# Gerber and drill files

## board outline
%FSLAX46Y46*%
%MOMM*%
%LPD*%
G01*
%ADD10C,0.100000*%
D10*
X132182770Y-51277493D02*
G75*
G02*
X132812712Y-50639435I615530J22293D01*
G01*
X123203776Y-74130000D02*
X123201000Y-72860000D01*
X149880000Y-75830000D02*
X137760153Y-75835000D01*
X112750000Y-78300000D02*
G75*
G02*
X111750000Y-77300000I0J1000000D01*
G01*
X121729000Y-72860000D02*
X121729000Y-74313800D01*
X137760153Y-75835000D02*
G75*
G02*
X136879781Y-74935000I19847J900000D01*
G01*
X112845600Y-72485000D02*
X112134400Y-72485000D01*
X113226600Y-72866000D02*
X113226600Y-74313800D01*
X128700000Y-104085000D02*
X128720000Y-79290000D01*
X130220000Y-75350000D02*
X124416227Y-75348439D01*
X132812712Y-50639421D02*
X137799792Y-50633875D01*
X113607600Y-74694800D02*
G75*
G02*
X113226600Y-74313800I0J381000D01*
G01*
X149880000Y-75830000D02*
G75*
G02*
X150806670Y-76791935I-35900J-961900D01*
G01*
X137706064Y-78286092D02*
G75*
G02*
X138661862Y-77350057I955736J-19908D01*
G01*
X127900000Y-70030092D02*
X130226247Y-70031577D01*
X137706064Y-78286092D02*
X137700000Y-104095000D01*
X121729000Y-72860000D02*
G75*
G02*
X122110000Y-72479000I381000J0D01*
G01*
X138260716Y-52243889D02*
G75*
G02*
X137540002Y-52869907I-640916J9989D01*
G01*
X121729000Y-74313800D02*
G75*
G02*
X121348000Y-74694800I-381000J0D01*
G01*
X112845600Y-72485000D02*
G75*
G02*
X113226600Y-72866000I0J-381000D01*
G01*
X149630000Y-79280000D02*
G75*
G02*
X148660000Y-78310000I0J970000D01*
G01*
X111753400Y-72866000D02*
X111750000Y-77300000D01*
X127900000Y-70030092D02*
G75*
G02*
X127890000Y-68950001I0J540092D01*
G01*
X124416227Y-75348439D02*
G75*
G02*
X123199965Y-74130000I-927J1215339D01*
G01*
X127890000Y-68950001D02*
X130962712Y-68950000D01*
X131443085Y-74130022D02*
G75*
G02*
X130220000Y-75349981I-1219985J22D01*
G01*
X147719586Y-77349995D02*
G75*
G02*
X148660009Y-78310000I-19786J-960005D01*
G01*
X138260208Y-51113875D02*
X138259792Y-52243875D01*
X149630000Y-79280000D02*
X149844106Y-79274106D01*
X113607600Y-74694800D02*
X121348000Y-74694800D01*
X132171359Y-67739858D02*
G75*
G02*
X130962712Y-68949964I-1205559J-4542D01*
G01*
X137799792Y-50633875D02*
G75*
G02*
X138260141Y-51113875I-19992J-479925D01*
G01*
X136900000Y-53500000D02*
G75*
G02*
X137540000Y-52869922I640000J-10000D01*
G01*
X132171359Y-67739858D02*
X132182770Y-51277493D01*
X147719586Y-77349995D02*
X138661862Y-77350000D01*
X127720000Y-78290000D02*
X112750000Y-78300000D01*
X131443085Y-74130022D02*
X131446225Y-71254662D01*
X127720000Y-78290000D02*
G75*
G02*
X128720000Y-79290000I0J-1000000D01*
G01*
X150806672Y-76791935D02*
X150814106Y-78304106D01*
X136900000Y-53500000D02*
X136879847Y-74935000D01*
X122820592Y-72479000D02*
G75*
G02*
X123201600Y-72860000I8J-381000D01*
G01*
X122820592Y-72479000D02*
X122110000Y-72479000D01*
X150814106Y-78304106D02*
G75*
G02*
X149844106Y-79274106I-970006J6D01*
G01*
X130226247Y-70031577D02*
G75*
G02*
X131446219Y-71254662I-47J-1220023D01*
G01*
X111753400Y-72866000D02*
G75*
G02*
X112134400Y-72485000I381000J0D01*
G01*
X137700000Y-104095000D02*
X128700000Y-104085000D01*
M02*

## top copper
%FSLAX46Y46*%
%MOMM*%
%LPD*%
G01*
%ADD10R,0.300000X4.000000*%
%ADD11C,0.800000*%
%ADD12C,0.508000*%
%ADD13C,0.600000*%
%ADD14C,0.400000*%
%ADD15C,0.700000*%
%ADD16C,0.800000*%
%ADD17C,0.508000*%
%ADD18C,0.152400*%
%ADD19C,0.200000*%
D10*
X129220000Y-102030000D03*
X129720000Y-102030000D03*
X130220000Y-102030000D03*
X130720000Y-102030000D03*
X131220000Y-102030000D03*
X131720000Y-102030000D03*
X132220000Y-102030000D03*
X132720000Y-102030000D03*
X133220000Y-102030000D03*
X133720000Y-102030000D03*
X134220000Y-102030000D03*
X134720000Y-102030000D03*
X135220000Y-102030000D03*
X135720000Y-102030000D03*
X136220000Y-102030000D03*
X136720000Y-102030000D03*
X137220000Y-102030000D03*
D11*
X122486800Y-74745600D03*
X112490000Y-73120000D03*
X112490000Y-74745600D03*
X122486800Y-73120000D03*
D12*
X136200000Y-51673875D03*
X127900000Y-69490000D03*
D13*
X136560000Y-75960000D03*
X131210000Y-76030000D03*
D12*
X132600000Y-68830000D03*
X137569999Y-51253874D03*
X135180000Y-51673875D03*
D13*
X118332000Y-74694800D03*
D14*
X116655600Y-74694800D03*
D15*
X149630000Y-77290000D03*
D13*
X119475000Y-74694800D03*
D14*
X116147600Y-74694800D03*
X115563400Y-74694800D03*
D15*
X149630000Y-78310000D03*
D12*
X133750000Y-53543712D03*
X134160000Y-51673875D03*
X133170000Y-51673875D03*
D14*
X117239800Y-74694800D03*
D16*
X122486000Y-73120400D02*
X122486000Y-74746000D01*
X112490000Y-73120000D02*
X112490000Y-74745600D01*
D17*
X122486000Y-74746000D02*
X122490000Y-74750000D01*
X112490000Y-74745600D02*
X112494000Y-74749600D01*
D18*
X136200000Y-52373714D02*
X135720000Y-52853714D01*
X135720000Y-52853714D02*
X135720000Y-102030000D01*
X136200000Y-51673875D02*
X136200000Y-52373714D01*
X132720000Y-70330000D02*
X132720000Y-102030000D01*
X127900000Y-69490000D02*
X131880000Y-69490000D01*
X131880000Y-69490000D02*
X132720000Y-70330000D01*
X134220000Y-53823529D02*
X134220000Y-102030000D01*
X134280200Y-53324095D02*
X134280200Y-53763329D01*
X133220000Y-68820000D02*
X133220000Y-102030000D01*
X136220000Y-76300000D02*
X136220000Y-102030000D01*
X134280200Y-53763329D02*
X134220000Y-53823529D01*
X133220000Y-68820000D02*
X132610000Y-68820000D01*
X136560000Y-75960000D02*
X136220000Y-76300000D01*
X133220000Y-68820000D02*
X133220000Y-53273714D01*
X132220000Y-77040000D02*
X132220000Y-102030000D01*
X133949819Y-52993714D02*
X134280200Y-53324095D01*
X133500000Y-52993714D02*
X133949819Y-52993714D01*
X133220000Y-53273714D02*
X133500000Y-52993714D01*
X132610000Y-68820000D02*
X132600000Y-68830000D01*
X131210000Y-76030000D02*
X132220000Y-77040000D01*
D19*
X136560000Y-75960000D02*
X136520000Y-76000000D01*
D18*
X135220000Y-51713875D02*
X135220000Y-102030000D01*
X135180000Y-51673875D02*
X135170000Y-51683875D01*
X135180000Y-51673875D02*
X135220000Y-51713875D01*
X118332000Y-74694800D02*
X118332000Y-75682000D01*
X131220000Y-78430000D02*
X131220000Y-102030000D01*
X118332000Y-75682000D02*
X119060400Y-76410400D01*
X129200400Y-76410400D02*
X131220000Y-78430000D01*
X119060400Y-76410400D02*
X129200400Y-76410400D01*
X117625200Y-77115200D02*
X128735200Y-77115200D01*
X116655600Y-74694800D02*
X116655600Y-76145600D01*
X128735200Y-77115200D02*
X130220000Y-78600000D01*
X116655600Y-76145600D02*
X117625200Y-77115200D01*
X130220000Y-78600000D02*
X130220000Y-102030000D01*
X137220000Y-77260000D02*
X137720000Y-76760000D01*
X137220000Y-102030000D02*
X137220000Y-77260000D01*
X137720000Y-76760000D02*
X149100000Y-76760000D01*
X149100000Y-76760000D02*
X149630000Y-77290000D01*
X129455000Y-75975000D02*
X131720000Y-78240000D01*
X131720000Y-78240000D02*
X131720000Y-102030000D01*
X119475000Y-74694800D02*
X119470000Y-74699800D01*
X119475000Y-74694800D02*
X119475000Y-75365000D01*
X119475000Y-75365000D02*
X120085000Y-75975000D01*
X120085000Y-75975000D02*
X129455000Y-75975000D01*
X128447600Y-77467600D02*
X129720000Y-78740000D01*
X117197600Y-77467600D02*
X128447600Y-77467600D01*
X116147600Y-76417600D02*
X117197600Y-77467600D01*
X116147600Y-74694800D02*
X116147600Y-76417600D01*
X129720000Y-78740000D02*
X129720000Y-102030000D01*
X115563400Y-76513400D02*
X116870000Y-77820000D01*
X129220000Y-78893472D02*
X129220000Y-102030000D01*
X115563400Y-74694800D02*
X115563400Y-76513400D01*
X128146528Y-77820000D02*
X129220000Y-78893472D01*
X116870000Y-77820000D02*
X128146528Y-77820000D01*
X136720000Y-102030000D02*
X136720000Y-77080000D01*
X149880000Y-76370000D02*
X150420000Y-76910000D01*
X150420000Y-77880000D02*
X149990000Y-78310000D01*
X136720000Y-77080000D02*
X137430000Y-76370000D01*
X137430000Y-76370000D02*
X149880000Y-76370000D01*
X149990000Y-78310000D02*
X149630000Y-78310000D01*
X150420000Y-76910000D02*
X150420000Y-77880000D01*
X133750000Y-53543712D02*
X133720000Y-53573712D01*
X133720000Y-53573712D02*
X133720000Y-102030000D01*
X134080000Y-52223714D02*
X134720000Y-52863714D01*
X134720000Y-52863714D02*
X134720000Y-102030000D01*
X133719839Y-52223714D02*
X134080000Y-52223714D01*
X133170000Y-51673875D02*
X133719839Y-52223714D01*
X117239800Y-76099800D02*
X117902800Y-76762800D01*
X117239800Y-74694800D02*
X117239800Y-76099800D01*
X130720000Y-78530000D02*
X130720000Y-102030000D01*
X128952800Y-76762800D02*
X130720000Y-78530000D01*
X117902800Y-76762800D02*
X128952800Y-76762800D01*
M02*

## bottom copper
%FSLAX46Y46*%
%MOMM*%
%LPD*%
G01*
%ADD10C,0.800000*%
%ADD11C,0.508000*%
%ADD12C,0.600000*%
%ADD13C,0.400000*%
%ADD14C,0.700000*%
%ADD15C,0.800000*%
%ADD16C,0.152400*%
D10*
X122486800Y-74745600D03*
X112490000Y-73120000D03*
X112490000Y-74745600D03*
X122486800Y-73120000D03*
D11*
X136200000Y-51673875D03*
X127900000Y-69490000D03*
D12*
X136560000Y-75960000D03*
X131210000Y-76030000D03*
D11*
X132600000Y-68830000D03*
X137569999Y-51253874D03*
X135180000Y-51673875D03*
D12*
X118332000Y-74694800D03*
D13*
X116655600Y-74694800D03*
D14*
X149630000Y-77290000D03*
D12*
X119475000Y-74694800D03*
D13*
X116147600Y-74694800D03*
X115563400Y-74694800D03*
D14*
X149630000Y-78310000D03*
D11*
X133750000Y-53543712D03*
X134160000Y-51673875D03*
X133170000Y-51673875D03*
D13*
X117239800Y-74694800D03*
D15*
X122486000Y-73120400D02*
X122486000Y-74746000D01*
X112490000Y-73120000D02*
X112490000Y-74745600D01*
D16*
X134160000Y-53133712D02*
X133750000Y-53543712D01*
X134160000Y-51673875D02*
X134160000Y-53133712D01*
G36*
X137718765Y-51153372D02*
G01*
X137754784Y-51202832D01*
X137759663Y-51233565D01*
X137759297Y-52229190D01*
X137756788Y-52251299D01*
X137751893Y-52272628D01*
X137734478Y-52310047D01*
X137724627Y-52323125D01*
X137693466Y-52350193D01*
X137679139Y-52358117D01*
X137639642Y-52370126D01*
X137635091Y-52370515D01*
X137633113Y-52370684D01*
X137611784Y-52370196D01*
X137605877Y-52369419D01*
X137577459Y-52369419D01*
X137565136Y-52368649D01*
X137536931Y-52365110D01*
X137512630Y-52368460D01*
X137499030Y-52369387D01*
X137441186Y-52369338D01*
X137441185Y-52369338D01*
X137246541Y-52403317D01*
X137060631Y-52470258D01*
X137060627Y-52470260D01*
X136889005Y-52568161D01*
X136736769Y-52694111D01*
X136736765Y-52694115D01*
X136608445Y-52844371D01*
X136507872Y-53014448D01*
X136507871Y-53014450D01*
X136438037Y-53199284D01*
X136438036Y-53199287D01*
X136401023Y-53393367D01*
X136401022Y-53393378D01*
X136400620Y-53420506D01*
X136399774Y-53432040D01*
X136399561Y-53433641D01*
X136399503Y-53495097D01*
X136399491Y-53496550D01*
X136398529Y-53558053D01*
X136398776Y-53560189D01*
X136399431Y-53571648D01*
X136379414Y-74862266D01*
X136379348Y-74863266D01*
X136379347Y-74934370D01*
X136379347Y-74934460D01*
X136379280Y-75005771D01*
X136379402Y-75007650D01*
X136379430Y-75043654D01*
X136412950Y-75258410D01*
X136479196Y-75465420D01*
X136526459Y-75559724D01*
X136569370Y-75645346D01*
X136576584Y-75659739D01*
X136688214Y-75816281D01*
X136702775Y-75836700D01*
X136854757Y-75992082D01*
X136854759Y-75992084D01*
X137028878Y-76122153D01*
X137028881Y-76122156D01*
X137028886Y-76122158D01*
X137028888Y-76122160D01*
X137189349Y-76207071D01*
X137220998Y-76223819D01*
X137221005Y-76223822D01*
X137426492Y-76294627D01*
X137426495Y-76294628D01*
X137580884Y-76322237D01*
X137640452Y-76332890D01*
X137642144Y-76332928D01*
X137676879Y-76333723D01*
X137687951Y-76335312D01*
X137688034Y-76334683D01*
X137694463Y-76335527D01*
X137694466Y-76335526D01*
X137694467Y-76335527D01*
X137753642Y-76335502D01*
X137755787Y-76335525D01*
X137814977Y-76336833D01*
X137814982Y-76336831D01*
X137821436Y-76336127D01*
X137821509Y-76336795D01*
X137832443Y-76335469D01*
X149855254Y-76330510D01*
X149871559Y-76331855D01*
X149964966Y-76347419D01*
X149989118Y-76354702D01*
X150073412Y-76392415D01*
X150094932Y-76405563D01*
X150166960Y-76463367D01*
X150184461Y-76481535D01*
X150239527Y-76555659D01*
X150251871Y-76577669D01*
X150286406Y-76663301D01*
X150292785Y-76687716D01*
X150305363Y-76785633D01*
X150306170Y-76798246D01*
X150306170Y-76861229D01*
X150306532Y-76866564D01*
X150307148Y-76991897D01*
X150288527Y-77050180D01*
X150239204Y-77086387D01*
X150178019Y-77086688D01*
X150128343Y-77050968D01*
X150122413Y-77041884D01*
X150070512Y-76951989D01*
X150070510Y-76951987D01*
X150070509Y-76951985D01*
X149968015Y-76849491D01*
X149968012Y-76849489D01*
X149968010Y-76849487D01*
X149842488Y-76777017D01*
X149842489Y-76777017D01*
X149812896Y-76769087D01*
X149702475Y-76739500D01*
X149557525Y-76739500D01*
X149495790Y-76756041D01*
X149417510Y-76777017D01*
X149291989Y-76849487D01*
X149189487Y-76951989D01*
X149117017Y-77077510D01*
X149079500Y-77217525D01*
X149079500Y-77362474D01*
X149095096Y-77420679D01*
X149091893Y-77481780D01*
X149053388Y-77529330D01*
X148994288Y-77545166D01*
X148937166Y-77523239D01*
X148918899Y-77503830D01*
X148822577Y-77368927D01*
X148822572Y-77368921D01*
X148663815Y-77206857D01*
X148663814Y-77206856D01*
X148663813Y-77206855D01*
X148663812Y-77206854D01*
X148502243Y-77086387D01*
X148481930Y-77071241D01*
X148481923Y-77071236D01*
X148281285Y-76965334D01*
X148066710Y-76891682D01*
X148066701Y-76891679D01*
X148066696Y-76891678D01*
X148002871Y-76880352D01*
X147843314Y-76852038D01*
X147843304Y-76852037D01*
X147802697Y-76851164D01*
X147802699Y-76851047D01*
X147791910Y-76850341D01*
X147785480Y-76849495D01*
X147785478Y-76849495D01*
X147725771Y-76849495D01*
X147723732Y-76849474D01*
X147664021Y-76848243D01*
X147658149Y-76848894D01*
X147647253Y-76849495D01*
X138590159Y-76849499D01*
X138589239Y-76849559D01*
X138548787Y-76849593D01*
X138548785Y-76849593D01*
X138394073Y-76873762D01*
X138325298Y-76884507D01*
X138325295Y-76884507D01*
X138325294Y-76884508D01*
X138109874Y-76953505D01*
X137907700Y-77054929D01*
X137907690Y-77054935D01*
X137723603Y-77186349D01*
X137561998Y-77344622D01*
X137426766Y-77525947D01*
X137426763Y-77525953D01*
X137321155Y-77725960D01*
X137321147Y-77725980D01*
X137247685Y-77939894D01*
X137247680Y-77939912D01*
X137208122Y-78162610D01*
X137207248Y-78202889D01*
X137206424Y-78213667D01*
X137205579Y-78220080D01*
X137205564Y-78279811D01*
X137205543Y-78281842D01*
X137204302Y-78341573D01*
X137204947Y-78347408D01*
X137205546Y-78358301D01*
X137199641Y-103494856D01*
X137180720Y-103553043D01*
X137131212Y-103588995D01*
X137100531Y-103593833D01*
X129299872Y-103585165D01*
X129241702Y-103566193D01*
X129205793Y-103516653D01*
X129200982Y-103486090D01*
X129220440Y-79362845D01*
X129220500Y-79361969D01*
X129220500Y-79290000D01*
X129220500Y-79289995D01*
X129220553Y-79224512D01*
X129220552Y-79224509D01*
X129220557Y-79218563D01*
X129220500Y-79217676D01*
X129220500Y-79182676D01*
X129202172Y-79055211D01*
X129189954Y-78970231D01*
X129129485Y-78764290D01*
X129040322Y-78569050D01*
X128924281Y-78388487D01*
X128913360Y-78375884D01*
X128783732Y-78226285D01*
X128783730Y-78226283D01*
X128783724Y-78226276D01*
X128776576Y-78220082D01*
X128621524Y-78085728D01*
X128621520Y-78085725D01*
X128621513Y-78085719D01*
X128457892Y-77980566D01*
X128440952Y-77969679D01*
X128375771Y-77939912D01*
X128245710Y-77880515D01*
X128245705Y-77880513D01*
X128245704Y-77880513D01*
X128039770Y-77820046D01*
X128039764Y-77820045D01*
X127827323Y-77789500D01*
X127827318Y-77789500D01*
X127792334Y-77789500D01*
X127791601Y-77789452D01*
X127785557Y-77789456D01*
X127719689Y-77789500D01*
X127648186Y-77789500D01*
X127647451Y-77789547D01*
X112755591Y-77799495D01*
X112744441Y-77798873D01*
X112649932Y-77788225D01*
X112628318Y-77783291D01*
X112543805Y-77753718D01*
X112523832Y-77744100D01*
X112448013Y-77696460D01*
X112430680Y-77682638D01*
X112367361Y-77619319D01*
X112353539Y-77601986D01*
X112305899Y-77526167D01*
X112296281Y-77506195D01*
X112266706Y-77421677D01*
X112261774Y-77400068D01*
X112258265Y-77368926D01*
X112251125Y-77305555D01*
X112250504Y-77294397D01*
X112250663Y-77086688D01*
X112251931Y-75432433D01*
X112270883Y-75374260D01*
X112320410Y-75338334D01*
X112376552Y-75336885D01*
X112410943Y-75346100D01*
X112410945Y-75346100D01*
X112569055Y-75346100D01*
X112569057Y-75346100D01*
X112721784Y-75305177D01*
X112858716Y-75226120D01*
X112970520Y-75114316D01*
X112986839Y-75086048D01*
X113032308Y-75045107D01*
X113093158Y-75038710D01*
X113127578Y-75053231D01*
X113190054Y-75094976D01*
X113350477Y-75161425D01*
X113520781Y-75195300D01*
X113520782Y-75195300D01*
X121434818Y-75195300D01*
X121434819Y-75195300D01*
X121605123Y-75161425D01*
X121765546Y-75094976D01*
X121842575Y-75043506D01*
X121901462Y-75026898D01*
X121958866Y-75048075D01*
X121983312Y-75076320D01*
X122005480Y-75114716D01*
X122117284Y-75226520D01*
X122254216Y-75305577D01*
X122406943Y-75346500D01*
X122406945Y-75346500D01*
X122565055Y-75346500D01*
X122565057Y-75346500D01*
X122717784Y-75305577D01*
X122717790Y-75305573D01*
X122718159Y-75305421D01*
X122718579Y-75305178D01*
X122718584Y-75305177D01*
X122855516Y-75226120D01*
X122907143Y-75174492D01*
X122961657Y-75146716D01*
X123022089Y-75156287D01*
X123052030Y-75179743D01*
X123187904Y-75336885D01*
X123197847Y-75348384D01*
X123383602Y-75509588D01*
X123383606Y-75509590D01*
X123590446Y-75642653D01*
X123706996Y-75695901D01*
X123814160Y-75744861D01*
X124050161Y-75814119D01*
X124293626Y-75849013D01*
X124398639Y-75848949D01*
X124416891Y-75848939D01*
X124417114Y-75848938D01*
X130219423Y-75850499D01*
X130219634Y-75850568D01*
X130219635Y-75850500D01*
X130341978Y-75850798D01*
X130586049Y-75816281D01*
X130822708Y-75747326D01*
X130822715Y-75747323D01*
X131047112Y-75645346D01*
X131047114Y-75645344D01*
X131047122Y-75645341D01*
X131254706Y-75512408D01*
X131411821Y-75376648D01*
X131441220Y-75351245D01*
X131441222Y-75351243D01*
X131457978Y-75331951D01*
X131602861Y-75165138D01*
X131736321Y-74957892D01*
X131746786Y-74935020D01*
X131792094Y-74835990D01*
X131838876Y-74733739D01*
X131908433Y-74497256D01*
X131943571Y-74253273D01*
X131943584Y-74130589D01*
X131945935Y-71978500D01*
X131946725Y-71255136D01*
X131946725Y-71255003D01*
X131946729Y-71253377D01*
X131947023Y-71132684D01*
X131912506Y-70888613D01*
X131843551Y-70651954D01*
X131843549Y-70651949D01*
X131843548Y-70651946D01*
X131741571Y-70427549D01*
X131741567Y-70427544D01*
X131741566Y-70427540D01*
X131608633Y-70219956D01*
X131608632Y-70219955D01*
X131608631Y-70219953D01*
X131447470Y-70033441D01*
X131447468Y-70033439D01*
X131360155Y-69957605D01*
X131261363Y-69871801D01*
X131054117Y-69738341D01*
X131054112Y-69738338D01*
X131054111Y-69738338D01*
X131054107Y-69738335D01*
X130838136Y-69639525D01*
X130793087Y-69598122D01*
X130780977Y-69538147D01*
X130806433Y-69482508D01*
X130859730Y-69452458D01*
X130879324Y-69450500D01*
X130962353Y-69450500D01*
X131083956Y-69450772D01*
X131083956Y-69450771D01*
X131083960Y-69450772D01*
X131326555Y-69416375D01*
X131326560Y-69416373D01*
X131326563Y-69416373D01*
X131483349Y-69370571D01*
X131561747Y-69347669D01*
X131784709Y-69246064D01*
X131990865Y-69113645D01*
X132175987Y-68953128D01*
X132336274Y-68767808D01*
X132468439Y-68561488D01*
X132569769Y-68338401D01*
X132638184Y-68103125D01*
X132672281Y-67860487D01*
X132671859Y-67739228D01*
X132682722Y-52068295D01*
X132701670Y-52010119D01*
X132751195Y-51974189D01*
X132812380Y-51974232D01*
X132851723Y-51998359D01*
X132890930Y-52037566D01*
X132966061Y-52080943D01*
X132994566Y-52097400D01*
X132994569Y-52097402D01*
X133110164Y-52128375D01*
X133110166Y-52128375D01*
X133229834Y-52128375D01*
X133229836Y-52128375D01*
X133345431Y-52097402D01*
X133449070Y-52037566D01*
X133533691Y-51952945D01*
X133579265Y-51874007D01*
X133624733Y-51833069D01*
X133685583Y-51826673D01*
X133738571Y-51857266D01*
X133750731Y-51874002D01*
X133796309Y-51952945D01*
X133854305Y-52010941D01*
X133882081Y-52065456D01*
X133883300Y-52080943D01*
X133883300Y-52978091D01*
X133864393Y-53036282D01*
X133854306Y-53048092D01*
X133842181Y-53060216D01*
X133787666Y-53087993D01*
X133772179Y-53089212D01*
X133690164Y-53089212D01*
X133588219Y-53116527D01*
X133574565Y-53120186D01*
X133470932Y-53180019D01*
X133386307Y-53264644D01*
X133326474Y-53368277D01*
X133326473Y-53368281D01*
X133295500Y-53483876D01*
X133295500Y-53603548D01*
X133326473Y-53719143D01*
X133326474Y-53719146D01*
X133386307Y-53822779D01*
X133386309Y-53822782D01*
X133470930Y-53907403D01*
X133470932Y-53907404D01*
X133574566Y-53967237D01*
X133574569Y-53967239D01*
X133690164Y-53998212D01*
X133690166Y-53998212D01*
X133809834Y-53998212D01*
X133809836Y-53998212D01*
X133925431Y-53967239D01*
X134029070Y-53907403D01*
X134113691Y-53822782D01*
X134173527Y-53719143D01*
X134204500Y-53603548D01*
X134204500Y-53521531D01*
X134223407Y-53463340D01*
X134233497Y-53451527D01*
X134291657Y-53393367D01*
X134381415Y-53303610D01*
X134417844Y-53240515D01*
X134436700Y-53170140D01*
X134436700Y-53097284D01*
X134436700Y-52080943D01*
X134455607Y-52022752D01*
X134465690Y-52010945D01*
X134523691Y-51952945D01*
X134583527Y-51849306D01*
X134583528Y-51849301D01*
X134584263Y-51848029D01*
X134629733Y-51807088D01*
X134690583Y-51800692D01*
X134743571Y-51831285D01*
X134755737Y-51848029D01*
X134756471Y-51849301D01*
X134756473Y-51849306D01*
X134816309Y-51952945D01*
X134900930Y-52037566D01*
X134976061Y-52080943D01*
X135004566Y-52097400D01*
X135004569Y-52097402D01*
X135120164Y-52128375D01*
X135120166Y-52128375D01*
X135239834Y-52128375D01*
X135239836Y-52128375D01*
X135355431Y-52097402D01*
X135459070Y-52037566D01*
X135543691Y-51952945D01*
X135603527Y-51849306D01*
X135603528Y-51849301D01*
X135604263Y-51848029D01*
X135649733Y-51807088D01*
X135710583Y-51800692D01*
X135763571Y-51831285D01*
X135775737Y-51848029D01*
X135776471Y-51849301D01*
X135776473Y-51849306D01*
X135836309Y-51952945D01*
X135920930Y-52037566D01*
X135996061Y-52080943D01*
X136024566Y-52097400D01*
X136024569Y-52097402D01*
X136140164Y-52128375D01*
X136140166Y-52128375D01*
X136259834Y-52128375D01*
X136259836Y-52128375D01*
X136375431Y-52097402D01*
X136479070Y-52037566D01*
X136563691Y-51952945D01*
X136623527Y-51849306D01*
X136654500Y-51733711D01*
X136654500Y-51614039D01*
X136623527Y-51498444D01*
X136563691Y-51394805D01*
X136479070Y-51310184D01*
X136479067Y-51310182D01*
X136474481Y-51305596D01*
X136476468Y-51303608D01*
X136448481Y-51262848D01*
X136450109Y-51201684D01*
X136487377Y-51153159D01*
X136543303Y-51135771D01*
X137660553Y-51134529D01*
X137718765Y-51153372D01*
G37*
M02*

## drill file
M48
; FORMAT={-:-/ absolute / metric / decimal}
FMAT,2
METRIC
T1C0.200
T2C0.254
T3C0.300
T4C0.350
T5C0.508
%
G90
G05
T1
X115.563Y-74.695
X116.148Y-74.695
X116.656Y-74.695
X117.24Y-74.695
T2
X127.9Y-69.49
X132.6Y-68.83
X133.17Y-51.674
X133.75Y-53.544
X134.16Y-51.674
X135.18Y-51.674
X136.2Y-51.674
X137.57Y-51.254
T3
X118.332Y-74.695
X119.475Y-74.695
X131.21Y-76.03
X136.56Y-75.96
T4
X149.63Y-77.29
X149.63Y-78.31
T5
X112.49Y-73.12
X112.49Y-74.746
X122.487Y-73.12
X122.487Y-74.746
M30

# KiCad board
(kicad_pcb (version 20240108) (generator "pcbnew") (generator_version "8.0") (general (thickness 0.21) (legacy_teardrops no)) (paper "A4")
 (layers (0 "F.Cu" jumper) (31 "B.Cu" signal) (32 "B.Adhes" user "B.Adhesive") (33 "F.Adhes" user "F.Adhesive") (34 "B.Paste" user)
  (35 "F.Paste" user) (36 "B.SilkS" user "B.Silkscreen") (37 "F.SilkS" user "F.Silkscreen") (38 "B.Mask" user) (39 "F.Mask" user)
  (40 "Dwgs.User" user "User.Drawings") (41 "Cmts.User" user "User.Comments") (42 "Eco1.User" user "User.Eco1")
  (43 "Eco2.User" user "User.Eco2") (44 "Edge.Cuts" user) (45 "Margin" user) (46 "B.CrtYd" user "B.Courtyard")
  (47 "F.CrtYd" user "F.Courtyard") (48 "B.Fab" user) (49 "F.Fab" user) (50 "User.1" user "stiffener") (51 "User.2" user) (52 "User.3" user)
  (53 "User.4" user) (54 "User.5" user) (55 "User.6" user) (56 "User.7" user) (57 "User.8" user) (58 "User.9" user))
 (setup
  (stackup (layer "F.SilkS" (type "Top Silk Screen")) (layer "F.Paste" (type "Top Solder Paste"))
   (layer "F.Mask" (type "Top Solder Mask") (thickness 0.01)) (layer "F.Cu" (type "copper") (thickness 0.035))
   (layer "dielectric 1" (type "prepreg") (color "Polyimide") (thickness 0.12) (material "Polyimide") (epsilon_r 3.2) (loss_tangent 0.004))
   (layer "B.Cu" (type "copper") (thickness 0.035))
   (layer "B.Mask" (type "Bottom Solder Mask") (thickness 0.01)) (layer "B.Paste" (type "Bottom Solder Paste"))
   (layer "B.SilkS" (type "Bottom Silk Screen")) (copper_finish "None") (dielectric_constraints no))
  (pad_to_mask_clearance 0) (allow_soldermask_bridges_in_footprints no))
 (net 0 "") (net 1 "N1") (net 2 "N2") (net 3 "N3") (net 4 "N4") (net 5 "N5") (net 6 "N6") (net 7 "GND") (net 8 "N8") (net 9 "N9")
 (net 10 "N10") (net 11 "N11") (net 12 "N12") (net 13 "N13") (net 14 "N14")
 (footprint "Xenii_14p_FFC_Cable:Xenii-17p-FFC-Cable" (layer "F.Cu") (at 129.22 102.03 90)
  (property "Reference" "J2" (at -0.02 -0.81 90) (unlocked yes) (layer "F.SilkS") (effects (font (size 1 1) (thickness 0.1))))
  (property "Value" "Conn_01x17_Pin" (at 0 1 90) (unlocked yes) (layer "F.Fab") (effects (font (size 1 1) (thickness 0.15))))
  (pad "1" smd rect (at 0 0 90) (size 4 0.3) (layers "F.Cu" "F.Paste" "F.Mask") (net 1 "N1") (thermal_bridge_angle 45))
  (pad "2" smd rect (at 0 0.5 90) (size 4 0.3) (layers "F.Cu" "F.Paste" "F.Mask") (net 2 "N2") (thermal_bridge_angle 45))
  (pad "3" smd rect (at 0 1 90) (size 4 0.3) (layers "F.Cu" "F.Paste" "F.Mask") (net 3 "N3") (thermal_bridge_angle 45))
  (pad "4" smd rect (at 0 1.5 90) (size 4 0.3) (layers "F.Cu" "F.Paste" "F.Mask") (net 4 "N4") (thermal_bridge_angle 45))
  (pad "5" smd rect (at 0 2 90) (size 4 0.3) (layers "F.Cu" "F.Paste" "F.Mask") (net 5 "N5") (thermal_bridge_angle 45))
  (pad "6" smd rect (at 0 2.5 90) (size 4 0.3) (layers "F.Cu" "F.Paste" "F.Mask") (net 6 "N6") (thermal_bridge_angle 45))
  (pad "7" smd rect (at 0 3 90) (size 4 0.3) (layers "F.Cu" "F.Paste" "F.Mask") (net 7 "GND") (thermal_bridge_angle 45))
  (pad "8" smd rect (at 0 3.5 90) (size 4 0.3) (layers "F.Cu" "F.Paste" "F.Mask") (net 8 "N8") (thermal_bridge_angle 45))
  (pad "9" smd rect (at 0 4 90) (size 4 0.3) (layers "F.Cu" "F.Paste" "F.Mask") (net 7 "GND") (thermal_bridge_angle 45))
  (pad "10" smd rect (at 0 4.5 90) (size 4 0.3) (layers "F.Cu" "F.Paste" "F.Mask") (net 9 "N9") (thermal_bridge_angle 45))
  (pad "11" smd rect (at 0 5 90) (size 4 0.3) (layers "F.Cu" "F.Paste" "F.Mask") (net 7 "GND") (thermal_bridge_angle 45))
  (pad "12" smd rect (at 0 5.5 90) (size 4 0.3) (layers "F.Cu" "F.Paste" "F.Mask") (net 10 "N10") (thermal_bridge_angle 45))
  (pad "13" smd rect (at 0 6 90) (size 4 0.3) (layers "F.Cu" "F.Paste" "F.Mask") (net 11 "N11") (thermal_bridge_angle 45))
  (pad "14" smd rect (at 0 6.5 90) (size 4 0.3) (layers "F.Cu" "F.Paste" "F.Mask") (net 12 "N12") (thermal_bridge_angle 45))
  (pad "15" smd rect (at 0 7 90) (size 4 0.3) (layers "F.Cu" "F.Paste" "F.Mask") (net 7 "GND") (thermal_bridge_angle 45))
  (pad "16" smd rect (at 0 7.5 90) (size 4 0.3) (layers "F.Cu" "F.Paste" "F.Mask") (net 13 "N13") (thermal_bridge_angle 45))
  (pad "17" smd rect (at 0 8 90) (size 4 0.3) (layers "F.Cu" "F.Paste" "F.Mask") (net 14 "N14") (thermal_bridge_angle 45)))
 (gr_arc (start 132.18277 51.277493) (mid 132.359996 50.822475) (end 132.812712 50.639421) (stroke (width 0.1) (type default))
  (layer "Edge.Cuts"))
 (gr_line (start 123.203776 74.13) (end 123.201 72.86) (stroke (width 0.1) (type default)) (layer "Edge.Cuts"))
 (gr_line (start 149.88 75.83) (end 137.760153 75.835) (stroke (width 0.1) (type default)) (layer "Edge.Cuts"))
 (gr_arc (start 112.75 78.3) (mid 112.042893 78.007107) (end 111.75 77.3) (stroke (width 0.1) (type default)) (layer "Edge.Cuts"))
 (gr_line (start 121.729 72.86) (end 121.729 74.3138) (stroke (width 0.1) (type default)) (layer "Edge.Cuts"))
 (gr_arc (start 137.760153 75.835) (mid 137.1365 75.564479) (end 136.879847 74.935) (stroke (width 0.1) (type default)) (layer "Edge.Cuts"))
 (gr_line (start 112.8456 72.485) (end 112.1344 72.485) (stroke (width 0.1) (type default)) (layer "Edge.Cuts"))
 (gr_line (start 113.2266 72.866) (end 113.2266 74.3138) (stroke (width 0.1) (type default)) (layer "Edge.Cuts"))
 (gr_line (start 128.7 104.085) (end 128.72 79.29) (stroke (width 0.1) (type default)) (layer "Edge.Cuts"))
 (gr_line (start 130.22 75.35) (end 124.416227 75.348439) (stroke (width 0.1) (type default)) (layer "Edge.Cuts"))
 (gr_line (start 132.812712 50.639421) (end 137.799792 50.633875) (stroke (width 0.1) (type default)) (layer "Edge.Cuts"))
 (gr_arc (start 113.6076 74.6948) (mid 113.338192 74.583208) (end 113.2266 74.3138) (stroke (width 0.1) (type default)) (layer "Edge.Cuts"))
 (gr_arc (start 149.88 75.83) (mid 150.537328 76.124086) (end 150.806672 76.791935) (stroke (width 0.1) (type default)) (layer "Edge.Cuts"))
 (gr_arc (start 137.706064 78.286092) (mid 137.992937 77.622986) (end 138.661862 77.35) (stroke (width 0.1) (type default))
  (layer "Edge.Cuts"))
 (gr_line (start 127.9 70.030092) (end 130.226247 70.031577) (stroke (width 0.1) (type default)) (layer "Edge.Cuts"))
 (gr_line (start 137.706064 78.286092) (end 137.7 104.095) (stroke (width 0.1) (type default)) (layer "Edge.Cuts"))
 (gr_arc (start 121.729 72.86) (mid 121.840592 72.590592) (end 122.11 72.479) (stroke (width 0.1) (type default)) (layer "Edge.Cuts"))
 (gr_arc (start 138.260716 52.243889) (mid 138.040147 52.717837) (end 137.54 52.869921) (stroke (width 0.1) (type default))
  (layer "Edge.Cuts"))
 (gr_arc (start 121.729 74.3138) (mid 121.617408 74.583208) (end 121.348 74.6948) (stroke (width 0.1) (type default)) (layer "Edge.Cuts"))
 (gr_arc (start 112.8456 72.485) (mid 113.115008 72.596592) (end 113.2266 72.866) (stroke (width 0.1) (type default)) (layer "Edge.Cuts"))
 (gr_arc (start 149.63 79.28) (mid 148.944106 78.995894) (end 148.66 78.31) (stroke (width 0.1) (type default)) (layer "Edge.Cuts"))
 (gr_line (start 111.7534 72.866) (end 111.75 77.3) (stroke (width 0.1) (type default)) (layer "Edge.Cuts"))
 (gr_arc (start 127.9 70.030092) (mid 127.359931 69.495) (end 127.89 68.950001) (stroke (width 0.1) (type default)) (layer "Edge.Cuts"))
 (gr_arc (start 124.416227 75.348439) (mid 123.555173 74.991698) (end 123.2 74.13) (stroke (width 0.1) (type default)) (layer "Edge.Cuts"))
 (gr_line (start 127.89 68.950001) (end 130.962712 68.95) (stroke (width 0.1) (type default)) (layer "Edge.Cuts"))
 (gr_arc (start 131.443085 74.130022) (mid 131.084662 74.993775) (end 130.22 75.35) (stroke (width 0.1) (type default)) (layer "Edge.Cuts"))
 (gr_arc (start 147.719586 77.349995) (mid 148.38573 77.638062) (end 148.66 78.31) (stroke (width 0.1) (type default)) (layer "Edge.Cuts"))
 (gr_line (start 138.260208 51.113875) (end 138.259792 52.243875) (stroke (width 0.1) (type default)) (layer "Edge.Cuts"))
 (gr_line (start 149.63 79.28) (end 149.844106 79.274106) (stroke (width 0.1) (type default)) (layer "Edge.Cuts"))
 (gr_line (start 113.6076 74.6948) (end 121.348 74.6948) (stroke (width 0.1) (type default)) (layer "Edge.Cuts"))
 (gr_arc (start 132.171359 67.739858) (mid 131.818778 68.59636) (end 130.962712 68.95) (stroke (width 0.1) (type default))
  (layer "Edge.Cuts"))
 (gr_arc (start 137.799792 50.633875) (mid 138.126516 50.78131) (end 138.260208 51.113875) (stroke (width 0.1) (type default))
  (layer "Edge.Cuts"))
 (gr_arc (start 136.9 53.5) (mid 137.090951 53.053884) (end 137.54 52.869922) (stroke (width 0.1) (type default)) (layer "Edge.Cuts"))
 (gr_line (start 132.171359 67.739858) (end 132.18277 51.277493) (stroke (width 0.1) (type default)) (layer "Edge.Cuts"))
 (gr_line (start 147.719586 77.349995) (end 138.661862 77.35) (stroke (width 0.1) (type default)) (layer "Edge.Cuts"))
 (gr_line (start 127.72 78.29) (end 112.75 78.3) (stroke (width 0.1) (type default)) (layer "Edge.Cuts"))
 (gr_line (start 131.443085 74.130022) (end 131.446225 71.254662) (stroke (width 0.1) (type default)) (layer "Edge.Cuts"))
 (gr_arc (start 127.72 78.29) (mid 128.427107 78.582893) (end 128.72 79.29) (stroke (width 0.1) (type default)) (layer "Edge.Cuts"))
 (gr_line (start 150.806672 76.791935) (end 150.814106 78.304106) (stroke (width 0.1) (type default)) (layer "Edge.Cuts"))
 (gr_line (start 136.9 53.5) (end 136.879847 74.935) (stroke (width 0.1) (type default)) (layer "Edge.Cuts"))
 (gr_arc (start 122.820592 72.479) (mid 123.09 72.590592) (end 123.201592 72.86) (stroke (width 0.1) (type default)) (layer "Edge.Cuts"))
 (gr_line (start 122.820592 72.479) (end 122.11 72.479) (stroke (width 0.1) (type default)) (layer "Edge.Cuts"))
 (gr_arc (start 150.814106 78.304106) (mid 150.529998 78.989998) (end 149.844106 79.274106) (stroke (width 0.1) (type default))
  (layer "Edge.Cuts"))
 (gr_arc (start 130.226247 70.031577) (mid 131.09 70.39) (end 131.446225 71.254662) (stroke (width 0.1) (type default)) (layer "Edge.Cuts"))
 (gr_arc (start 111.7534 72.866) (mid 111.864992 72.596592) (end 112.1344 72.485) (stroke (width 0.1) (type default)) (layer "Edge.Cuts"))
 (gr_line (start 137.7 104.095) (end 128.7 104.085) (stroke (width 0.1) (type default)) (layer "Edge.Cuts"))
 (segment (start 122.486 73.1204) (end 122.486 74.746) (width 0.8) (layer "F.Cu") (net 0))
 (segment (start 112.49 73.12) (end 112.49 74.7456) (width 0.8) (layer "F.Cu") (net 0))
 (segment (start 122.486 74.746) (end 122.49 74.75) (width 0.508) (layer "F.Cu") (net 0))
 (segment (start 112.49 74.7456) (end 112.494 74.7496) (width 0.508) (layer "F.Cu") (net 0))
 (via (at 122.4868 74.7456) (size 0.8) (drill 0.508) (layers "F.Cu" "B.Cu") (free yes) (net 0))
 (via (at 112.49 73.12) (size 0.8) (drill 0.508) (layers "F.Cu" "B.Cu") (free yes) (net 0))
 (via (at 112.49 74.7456) (size 0.8) (drill 0.508) (layers "F.Cu" "B.Cu") (free yes) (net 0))
 (via (at 122.4868 73.12) (size 0.8) (drill 0.508) (layers "F.Cu" "B.Cu") (free yes) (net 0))
 (segment (start 122.486 73.1204) (end 122.486 74.746) (width 0.8) (layer "B.Cu") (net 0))
 (segment (start 112.49 73.12) (end 112.49 74.7456) (width 0.8) (layer "B.Cu") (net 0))
 (segment (start 136.2 52.373714) (end 135.72 52.853714) (width 0.1524) (layer "F.Cu") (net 12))
 (segment (start 135.72 52.853714) (end 135.72 102.03) (width 0.1524) (layer "F.Cu") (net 12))
 (segment (start 136.2 51.673875) (end 136.2 52.373714) (width 0.1524) (layer "F.Cu") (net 12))
 (via (at 136.2 51.673875) (size 0.508) (drill 0.254253) (layers "F.Cu" "B.Cu") (free yes) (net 12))
 (segment (start 132.72 70.33) (end 132.72 102.03) (width 0.1524) (layer "F.Cu") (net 8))
 (segment (start 127.9 69.49) (end 131.88 69.49) (width 0.1524) (layer "F.Cu") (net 8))
 (segment (start 131.88 69.49) (end 132.72 70.33) (width 0.1524) (layer "F.Cu") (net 8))
 (via (at 127.9 69.49) (size 0.508) (drill 0.254253) (layers "F.Cu" "B.Cu") (free yes) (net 8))
 (segment (start 134.22 53.823529) (end 134.22 102.03) (width 0.1524) (layer "F.Cu") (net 7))
 (segment (start 134.2802 53.324095) (end 134.2802 53.763329) (width 0.1524) (layer "F.Cu") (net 7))
 (segment (start 133.22 68.82) (end 133.22 102.03) (width 0.1524) (layer "F.Cu") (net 7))
 (segment (start 136.22 76.3) (end 136.22 102.03) (width 0.1524) (layer "F.Cu") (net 7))
 (segment (start 134.2802 53.763329) (end 134.22 53.823529) (width 0.1524) (layer "F.Cu") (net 7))
 (segment (start 133.22 68.82) (end 132.61 68.82) (width 0.1524) (layer "F.Cu") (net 7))
 (segment (start 136.56 75.96) (end 136.22 76.3) (width 0.1524) (layer "F.Cu") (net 7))
 (segment (start 133.22 68.82) (end 133.22 53.273714) (width 0.1524) (layer "F.Cu") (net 7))
 (segment (start 132.22 77.04) (end 132.22 102.03) (width 0.1524) (layer "F.Cu") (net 7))
 (segment (start 133.949819 52.993714) (end 134.2802 53.324095) (width 0.1524) (layer "F.Cu") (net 7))
 (segment (start 133.5 52.993714) (end 133.949819 52.993714) (width 0.1524) (layer "F.Cu") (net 7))
 (segment (start 133.22 53.273714) (end 133.5 52.993714) (width 0.1524) (layer "F.Cu") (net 7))
 (segment (start 132.61 68.82) (end 132.6 68.83) (width 0.1524) (layer "F.Cu") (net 7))
 (segment (start 131.21 76.03) (end 132.22 77.04) (width 0.1524) (layer "F.Cu") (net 7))
 (segment (start 136.56 75.96) (end 136.52 76) (width 0.2) (layer "F.Cu") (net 7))
 (via (at 136.56 75.96) (size 0.6) (drill 0.3) (layers "F.Cu" "B.Cu") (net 7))
 (via (at 131.21 76.03) (size 0.6) (drill 0.3) (layers "F.Cu" "B.Cu") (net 7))
 (via (at 132.6 68.83) (size 0.508) (drill 0.254253) (layers "F.Cu" "B.Cu") (free yes) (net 7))
 (via (at 137.569999 51.253874) (size 0.508) (drill 0.254253) (layers "F.Cu" "B.Cu") (free yes) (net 7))
 (segment (start 135.22 51.713875) (end 135.22 102.03) (width 0.1524) (layer "F.Cu") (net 11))
 (segment (start 135.18 51.673875) (end 135.17 51.683875) (width 0.1524) (layer "F.Cu") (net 11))
 (segment (start 135.18 51.673875) (end 135.22 51.713875) (width 0.1524) (layer "F.Cu") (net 11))
 (via (at 135.18 51.673875) (size 0.508) (drill 0.254253) (layers "F.Cu" "B.Cu") (free yes) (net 11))
 (segment (start 118.332 74.6948) (end 118.332 75.682) (width 0.1524) (layer "F.Cu") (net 5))
 (segment (start 131.22 78.43) (end 131.22 102.03) (width 0.1524) (layer "F.Cu") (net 5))
 (segment (start 118.332 75.682) (end 119.0604 76.4104) (width 0.1524) (layer "F.Cu") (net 5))
 (segment (start 129.2004 76.4104) (end 131.22 78.43) (width 0.1524) (layer "F.Cu") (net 5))
 (segment (start 119.0604 76.4104) (end 129.2004 76.4104) (width 0.1524) (layer "F.Cu") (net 5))
 (via (at 118.332 74.6948) (size 0.6) (drill 0.3) (layers "F.Cu" "B.Cu") (free yes) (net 5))
 (segment (start 117.6252 77.1152) (end 128.7352 77.1152) (width 0.1524) (layer "F.Cu") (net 3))
 (segment (start 116.6556 74.6948) (end 116.6556 76.1456) (width 0.1524) (layer "F.Cu") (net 3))
 (segment (start 128.7352 77.1152) (end 130.22 78.6) (width 0.1524) (layer "F.Cu") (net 3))
 (segment (start 116.6556 76.1456) (end 117.6252 77.1152) (width 0.1524) (layer "F.Cu") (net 3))
 (segment (start 130.22 78.6) (end 130.22 102.03) (width 0.1524) (layer "F.Cu") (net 3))
 (via (at 116.6556 74.6948) (size 0.4) (drill 0.2) (layers "F.Cu" "B.Cu") (free yes) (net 3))
 (segment (start 137.22 77.26) (end 137.72 76.76) (width 0.1524) (layer "F.Cu") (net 14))
 (segment (start 137.22 102.03) (end 137.22 77.26) (width 0.1524) (layer "F.Cu") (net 14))
 (segment (start 137.72 76.76) (end 149.1 76.76) (width 0.1524) (layer "F.Cu") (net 14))
 (segment (start 149.1 76.76) (end 149.63 77.29) (width 0.1524) (layer "F.Cu") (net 14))
 (via (at 149.63 77.29) (size 0.7) (drill 0.35) (layers "F.Cu" "B.Cu") (free yes) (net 14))
 (segment (start 129.455 75.975) (end 131.72 78.24) (width 0.1524) (layer "F.Cu") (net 6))
 (segment (start 131.72 78.24) (end 131.72 102.03) (width 0.1524) (layer "F.Cu") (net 6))
 (segment (start 119.475 74.6948) (end 119.47 74.6998) (width 0.1524) (layer "F.Cu") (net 6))
 (segment (start 119.475 74.6948) (end 119.475 75.365) (width 0.1524) (layer "F.Cu") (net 6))
 (segment (start 119.475 75.365) (end 120.085 75.975) (width 0.1524) (layer "F.Cu") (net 6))
 (segment (start 120.085 75.975) (end 129.455 75.975) (width 0.1524) (layer "F.Cu") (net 6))
 (via (at 119.475 74.6948) (size 0.6) (drill 0.3) (layers "F.Cu" "B.Cu") (free yes) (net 6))
 (segment (start 128.4476 77.4676) (end 129.72 78.74) (width 0.1524) (layer "F.Cu") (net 2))
 (segment (start 117.1976 77.4676) (end 128.4476 77.4676) (width 0.1524) (layer "F.Cu") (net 2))
 (segment (start 116.1476 76.4176) (end 117.1976 77.4676) (width 0.1524) (layer "F.Cu") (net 2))
 (segment (start 116.1476 74.6948) (end 116.1476 76.4176) (width 0.1524) (layer "F.Cu") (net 2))
 (segment (start 129.72 78.74) (end 129.72 102.03) (width 0.1524) (layer "F.Cu") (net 2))
 (via (at 116.1476 74.6948) (size 0.4) (drill 0.2) (layers "F.Cu" "B.Cu") (free yes) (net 2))
 (segment (start 115.5634 76.5134) (end 116.87 77.82) (width 0.1524) (layer "F.Cu") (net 1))
 (segment (start 129.22 78.893472) (end 129.22 102.03) (width 0.1524) (layer "F.Cu") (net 1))
 (segment (start 115.5634 74.6948) (end 115.5634 76.5134) (width 0.1524) (layer "F.Cu") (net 1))
 (segment (start 128.146528 77.82) (end 129.22 78.893472) (width 0.1524) (layer "F.Cu") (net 1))
 (segment (start 116.87 77.82) (end 128.146528 77.82) (width 0.1524) (layer "F.Cu") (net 1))
 (via (at 115.5634 74.6948) (size 0.4) (drill 0.2) (layers "F.Cu" "B.Cu") (free yes) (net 1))
 (segment (start 136.72 102.03) (end 136.72 77.08) (width 0.1524) (layer "F.Cu") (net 13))
 (segment (start 149.88 76.37) (end 150.42 76.91) (width 0.1524) (layer "F.Cu") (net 13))
 (segment (start 150.42 77.88) (end 149.99 78.31) (width 0.1524) (layer "F.Cu") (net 13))
 (segment (start 136.72 77.08) (end 137.43 76.37) (width 0.1524) (layer "F.Cu") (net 13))
 (segment (start 137.43 76.37) (end 149.88 76.37) (width 0.1524) (layer "F.Cu") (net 13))
 (segment (start 149.99 78.31) (end 149.63 78.31) (width 0.1524) (layer "F.Cu") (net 13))
 (segment (start 150.42 76.91) (end 150.42 77.88) (width 0.1524) (layer "F.Cu") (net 13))
 (via (at 149.63 78.31) (size 0.7) (drill 0.35) (layers "F.Cu" "B.Cu") (free yes) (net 13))
 (segment (start 133.75 53.543712) (end 133.72 53.573712) (width 0.1524) (layer "F.Cu") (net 9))
 (segment (start 133.72 53.573712) (end 133.72 102.03) (width 0.1524) (layer "F.Cu") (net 9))
 (via (at 133.75 53.543712) (size 0.508) (drill 0.254253) (layers "F.Cu" "B.Cu") (free yes) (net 9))
 (via (at 134.16 51.673875) (size 0.508) (drill 0.254253) (layers "F.Cu" "B.Cu") (free yes) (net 9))
 (segment (start 134.16 53.133712) (end 133.75 53.543712) (width 0.1524) (layer "B.Cu") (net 9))
 (segment (start 134.16 51.673875) (end 134.16 53.133712) (width 0.1524) (layer "B.Cu") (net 9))
 (segment (start 134.08 52.223714) (end 134.72 52.863714) (width 0.1524) (layer "F.Cu") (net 10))
 (segment (start 134.72 52.863714) (end 134.72 102.03) (width 0.1524) (layer "F.Cu") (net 10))
 (segment (start 133.719839 52.223714) (end 134.08 52.223714) (width 0.1524) (layer "F.Cu") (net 10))
 (segment (start 133.17 51.673875) (end 133.719839 52.223714) (width 0.1524) (layer "F.Cu") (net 10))
 (via (at 133.17 51.673875) (size 0.508) (drill 0.254253) (layers "F.Cu" "B.Cu") (free yes) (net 10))
 (segment (start 117.2398 76.0998) (end 117.9028 76.7628) (width 0.1524) (layer "F.Cu") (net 4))
 (segment (start 117.2398 74.6948) (end 117.2398 76.0998) (width 0.1524) (layer "F.Cu") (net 4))
 (segment (start 130.72 78.53) (end 130.72 102.03) (width 0.1524) (layer "F.Cu") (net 4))
 (segment (start 128.9528 76.7628) (end 130.72 78.53) (width 0.1524) (layer "F.Cu") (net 4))
 (segment (start 117.9028 76.7628) (end 128.9528 76.7628) (width 0.1524) (layer "F.Cu") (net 4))
 (via (at 117.2398 74.6948) (size 0.4) (drill 0.2) (layers "F.Cu" "B.Cu") (free yes) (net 4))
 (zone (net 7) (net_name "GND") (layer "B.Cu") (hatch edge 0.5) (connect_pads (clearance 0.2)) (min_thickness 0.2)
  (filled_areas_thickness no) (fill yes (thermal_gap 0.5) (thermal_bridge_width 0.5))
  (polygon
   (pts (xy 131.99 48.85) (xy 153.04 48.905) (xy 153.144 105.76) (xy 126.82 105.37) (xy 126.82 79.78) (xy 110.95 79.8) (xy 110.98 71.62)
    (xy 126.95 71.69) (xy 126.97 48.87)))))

